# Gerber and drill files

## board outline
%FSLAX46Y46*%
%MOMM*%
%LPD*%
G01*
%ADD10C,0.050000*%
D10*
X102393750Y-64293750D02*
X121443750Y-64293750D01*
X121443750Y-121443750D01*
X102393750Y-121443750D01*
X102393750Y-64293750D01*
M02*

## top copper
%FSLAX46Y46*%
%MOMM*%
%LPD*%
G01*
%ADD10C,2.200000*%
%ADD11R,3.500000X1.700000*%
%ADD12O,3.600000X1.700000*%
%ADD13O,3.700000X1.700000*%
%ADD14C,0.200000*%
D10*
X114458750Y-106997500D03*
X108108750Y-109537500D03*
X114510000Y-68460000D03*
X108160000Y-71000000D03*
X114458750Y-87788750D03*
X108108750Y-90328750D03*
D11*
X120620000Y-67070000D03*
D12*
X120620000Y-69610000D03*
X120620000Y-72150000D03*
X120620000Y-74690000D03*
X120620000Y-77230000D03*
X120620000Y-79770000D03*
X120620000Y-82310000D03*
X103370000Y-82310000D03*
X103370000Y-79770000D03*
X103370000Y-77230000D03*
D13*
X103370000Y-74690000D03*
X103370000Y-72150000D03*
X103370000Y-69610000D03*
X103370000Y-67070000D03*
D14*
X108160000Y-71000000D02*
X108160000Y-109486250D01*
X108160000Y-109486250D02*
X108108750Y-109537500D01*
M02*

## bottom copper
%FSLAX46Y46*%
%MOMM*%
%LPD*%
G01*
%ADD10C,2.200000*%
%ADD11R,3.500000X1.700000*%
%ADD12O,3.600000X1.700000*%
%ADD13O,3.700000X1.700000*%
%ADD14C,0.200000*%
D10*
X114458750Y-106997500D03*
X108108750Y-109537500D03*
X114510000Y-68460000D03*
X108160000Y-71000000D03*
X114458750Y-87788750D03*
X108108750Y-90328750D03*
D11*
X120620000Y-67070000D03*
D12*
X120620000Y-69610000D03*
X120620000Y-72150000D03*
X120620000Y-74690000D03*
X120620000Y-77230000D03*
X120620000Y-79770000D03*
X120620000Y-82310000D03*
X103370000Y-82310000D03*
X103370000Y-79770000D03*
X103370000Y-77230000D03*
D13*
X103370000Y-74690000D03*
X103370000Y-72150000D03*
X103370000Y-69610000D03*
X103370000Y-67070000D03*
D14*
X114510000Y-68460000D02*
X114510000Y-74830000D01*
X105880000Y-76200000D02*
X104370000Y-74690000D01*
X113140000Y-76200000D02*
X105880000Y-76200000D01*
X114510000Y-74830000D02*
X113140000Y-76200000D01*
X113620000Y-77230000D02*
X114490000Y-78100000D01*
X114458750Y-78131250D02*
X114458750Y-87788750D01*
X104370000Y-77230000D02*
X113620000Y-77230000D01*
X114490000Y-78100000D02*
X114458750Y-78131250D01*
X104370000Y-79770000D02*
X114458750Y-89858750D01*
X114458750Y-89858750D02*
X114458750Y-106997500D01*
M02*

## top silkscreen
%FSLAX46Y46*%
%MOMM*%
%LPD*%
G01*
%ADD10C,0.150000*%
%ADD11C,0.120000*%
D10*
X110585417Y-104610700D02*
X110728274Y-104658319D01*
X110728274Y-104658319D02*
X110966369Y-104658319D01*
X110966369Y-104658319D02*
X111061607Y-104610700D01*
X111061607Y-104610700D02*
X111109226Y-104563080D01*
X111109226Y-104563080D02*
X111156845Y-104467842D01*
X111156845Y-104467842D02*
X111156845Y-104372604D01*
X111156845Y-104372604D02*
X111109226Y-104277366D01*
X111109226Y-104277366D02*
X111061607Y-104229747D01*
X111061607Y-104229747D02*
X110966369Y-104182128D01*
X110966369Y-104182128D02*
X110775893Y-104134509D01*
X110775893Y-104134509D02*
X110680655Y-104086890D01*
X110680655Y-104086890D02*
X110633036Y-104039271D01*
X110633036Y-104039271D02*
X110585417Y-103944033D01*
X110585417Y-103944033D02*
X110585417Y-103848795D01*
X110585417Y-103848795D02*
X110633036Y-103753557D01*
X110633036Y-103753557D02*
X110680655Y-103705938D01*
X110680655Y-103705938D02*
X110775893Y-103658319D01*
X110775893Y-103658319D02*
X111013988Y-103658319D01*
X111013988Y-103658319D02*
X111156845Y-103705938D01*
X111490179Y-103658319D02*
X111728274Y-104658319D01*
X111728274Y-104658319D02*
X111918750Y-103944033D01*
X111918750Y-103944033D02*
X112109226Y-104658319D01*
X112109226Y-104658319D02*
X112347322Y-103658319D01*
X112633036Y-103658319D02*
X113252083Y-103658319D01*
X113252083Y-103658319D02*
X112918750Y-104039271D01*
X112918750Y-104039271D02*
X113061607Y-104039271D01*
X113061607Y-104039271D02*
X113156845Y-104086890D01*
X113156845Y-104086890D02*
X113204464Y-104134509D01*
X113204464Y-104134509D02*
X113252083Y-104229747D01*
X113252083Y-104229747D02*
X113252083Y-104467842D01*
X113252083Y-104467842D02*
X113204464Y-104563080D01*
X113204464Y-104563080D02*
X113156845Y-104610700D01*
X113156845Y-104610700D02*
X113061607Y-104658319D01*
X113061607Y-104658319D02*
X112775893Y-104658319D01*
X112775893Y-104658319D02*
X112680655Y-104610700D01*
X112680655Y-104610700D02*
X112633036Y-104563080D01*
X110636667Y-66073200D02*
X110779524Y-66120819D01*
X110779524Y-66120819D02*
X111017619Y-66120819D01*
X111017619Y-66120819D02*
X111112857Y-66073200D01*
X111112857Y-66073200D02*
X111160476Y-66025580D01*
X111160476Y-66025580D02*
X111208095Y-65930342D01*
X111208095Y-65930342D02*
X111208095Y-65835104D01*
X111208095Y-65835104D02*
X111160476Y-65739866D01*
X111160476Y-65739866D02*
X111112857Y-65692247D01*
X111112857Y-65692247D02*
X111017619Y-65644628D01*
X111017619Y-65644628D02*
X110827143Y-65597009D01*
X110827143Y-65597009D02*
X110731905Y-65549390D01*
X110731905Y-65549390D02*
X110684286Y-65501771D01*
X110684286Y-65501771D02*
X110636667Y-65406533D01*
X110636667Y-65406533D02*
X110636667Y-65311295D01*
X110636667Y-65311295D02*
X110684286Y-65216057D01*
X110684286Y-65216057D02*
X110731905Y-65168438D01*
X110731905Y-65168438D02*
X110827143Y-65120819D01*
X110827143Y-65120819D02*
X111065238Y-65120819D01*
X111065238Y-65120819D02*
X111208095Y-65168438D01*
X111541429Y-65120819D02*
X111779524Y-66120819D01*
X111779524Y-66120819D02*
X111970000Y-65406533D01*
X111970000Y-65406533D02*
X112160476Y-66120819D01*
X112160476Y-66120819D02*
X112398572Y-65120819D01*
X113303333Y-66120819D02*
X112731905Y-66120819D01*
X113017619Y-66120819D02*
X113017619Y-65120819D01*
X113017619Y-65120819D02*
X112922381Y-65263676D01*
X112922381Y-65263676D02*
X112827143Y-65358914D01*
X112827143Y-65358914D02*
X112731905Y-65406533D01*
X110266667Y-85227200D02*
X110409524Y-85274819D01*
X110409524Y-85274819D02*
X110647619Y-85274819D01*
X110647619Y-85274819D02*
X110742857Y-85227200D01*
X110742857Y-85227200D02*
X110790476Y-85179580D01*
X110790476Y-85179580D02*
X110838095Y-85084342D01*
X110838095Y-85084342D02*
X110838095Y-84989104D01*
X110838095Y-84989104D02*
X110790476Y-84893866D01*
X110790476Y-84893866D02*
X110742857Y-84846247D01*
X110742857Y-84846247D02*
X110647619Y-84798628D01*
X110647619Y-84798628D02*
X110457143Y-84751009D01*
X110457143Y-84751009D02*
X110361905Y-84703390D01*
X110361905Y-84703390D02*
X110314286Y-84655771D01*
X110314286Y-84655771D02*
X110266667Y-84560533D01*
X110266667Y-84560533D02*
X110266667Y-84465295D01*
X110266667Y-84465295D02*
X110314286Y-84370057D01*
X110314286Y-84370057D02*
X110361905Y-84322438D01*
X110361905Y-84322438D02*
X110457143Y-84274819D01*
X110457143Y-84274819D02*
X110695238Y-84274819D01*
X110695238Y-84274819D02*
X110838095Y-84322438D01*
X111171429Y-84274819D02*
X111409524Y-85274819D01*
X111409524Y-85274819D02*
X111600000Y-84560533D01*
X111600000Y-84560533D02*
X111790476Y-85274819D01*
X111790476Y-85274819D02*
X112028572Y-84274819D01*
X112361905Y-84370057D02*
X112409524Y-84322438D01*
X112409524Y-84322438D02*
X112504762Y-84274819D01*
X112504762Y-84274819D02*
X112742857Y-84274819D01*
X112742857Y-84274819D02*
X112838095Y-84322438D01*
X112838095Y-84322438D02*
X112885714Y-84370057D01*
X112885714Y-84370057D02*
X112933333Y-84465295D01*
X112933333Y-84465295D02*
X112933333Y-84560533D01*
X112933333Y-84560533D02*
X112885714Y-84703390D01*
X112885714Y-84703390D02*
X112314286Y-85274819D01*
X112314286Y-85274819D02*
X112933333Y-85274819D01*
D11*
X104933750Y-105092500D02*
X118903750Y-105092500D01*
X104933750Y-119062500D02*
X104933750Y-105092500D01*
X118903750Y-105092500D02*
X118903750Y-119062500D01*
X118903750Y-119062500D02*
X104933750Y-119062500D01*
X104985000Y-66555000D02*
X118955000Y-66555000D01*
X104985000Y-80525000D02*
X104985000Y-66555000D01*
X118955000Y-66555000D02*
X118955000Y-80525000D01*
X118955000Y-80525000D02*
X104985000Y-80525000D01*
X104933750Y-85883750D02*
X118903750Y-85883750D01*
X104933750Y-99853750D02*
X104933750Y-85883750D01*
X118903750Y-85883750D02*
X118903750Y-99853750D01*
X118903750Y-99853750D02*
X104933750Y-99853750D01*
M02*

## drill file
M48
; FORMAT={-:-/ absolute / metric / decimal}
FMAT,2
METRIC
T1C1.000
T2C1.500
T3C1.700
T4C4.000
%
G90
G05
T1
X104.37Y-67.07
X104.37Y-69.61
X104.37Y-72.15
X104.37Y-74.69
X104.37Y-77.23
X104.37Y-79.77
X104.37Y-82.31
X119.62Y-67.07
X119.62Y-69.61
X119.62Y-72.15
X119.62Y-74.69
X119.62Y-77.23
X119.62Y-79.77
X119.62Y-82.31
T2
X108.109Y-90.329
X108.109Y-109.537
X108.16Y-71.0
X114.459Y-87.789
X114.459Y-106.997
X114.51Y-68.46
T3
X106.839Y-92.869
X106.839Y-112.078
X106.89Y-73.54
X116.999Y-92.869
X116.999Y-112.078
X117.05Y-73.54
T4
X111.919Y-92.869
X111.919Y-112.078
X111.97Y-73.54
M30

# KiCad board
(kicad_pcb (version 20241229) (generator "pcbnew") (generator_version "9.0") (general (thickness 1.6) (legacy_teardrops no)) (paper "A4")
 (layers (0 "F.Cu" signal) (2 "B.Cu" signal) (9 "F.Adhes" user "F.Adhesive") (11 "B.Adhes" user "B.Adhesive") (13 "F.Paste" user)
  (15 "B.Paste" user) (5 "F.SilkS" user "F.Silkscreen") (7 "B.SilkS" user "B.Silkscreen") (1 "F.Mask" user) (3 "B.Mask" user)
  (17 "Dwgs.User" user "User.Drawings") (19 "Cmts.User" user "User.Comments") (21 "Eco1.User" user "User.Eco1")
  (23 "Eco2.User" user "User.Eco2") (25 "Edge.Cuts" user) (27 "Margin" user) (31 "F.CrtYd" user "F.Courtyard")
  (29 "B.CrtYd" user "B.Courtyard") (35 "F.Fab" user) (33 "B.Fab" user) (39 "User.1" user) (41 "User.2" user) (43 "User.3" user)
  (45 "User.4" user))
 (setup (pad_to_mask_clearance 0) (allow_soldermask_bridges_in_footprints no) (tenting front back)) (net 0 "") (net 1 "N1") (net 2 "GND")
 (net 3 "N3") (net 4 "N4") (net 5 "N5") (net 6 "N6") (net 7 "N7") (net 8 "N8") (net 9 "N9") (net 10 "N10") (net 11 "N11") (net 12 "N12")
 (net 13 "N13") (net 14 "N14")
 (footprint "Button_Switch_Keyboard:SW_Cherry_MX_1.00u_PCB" (layer "F.Cu") (at 114.45875 106.9975)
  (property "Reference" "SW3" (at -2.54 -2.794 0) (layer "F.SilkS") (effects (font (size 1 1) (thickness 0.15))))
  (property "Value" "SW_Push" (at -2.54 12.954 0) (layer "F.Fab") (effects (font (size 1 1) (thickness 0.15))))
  (fp_line (start -9.525 -1.905) (end 4.445 -1.905) (stroke (width 0.12) (type solid)) (layer "F.SilkS"))
  (fp_line (start -9.525 12.065) (end -9.525 -1.905) (stroke (width 0.12) (type solid)) (layer "F.SilkS"))
  (fp_line (start 4.445 -1.905) (end 4.445 12.065) (stroke (width 0.12) (type solid)) (layer "F.SilkS"))
  (fp_line (start 4.445 12.065) (end -9.525 12.065) (stroke (width 0.12) (type solid)) (layer "F.SilkS"))
  (pad "" np_thru_hole circle (at -7.62 5.08) (size 1.7 1.7) (drill 1.7) (layers "*.Cu" "*.Mask"))
  (pad "" np_thru_hole circle (at -2.54 5.08) (size 4 4) (drill 4) (layers "*.Cu" "*.Mask"))
  (pad "" np_thru_hole circle (at 2.54 5.08) (size 1.7 1.7) (drill 1.7) (layers "*.Cu" "*.Mask"))
  (pad "1" thru_hole circle (at 0 0) (size 2.2 2.2) (drill 1.5) (layers "*.Cu" "*.Mask") (remove_unused_layers no) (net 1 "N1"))
  (pad "2" thru_hole circle (at -6.35 2.54) (size 2.2 2.2) (drill 1.5) (layers "*.Cu" "*.Mask") (remove_unused_layers no) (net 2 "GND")))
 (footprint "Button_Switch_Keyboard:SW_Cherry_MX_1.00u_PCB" (layer "F.Cu") (at 114.51 68.46)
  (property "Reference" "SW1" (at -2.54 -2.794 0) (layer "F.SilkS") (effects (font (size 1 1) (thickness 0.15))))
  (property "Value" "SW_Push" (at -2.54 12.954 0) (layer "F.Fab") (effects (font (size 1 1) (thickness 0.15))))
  (fp_line (start -9.525 -1.905) (end 4.445 -1.905) (stroke (width 0.12) (type solid)) (layer "F.SilkS"))
  (fp_line (start -9.525 12.065) (end -9.525 -1.905) (stroke (width 0.12) (type solid)) (layer "F.SilkS"))
  (fp_line (start 4.445 -1.905) (end 4.445 12.065) (stroke (width 0.12) (type solid)) (layer "F.SilkS"))
  (fp_line (start 4.445 12.065) (end -9.525 12.065) (stroke (width 0.12) (type solid)) (layer "F.SilkS"))
  (pad "" np_thru_hole circle (at -7.62 5.08) (size 1.7 1.7) (drill 1.7) (layers "*.Cu" "*.Mask"))
  (pad "" np_thru_hole circle (at -2.54 5.08) (size 4 4) (drill 4) (layers "*.Cu" "*.Mask"))
  (pad "" np_thru_hole circle (at 2.54 5.08) (size 1.7 1.7) (drill 1.7) (layers "*.Cu" "*.Mask"))
  (pad "1" thru_hole circle (at 0 0) (size 2.2 2.2) (drill 1.5) (layers "*.Cu" "*.Mask") (remove_unused_layers no) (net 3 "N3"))
  (pad "2" thru_hole circle (at -6.35 2.54) (size 2.2 2.2) (drill 1.5) (layers "*.Cu" "*.Mask") (remove_unused_layers no) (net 2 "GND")))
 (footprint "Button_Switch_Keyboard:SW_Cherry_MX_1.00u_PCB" (layer "F.Cu") (at 114.45875 87.78875)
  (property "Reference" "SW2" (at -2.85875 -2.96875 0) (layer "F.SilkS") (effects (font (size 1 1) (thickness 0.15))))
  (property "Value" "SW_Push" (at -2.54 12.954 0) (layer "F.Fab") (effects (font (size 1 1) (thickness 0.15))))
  (fp_line (start -9.525 -1.905) (end 4.445 -1.905) (stroke (width 0.12) (type solid)) (layer "F.SilkS"))
  (fp_line (start -9.525 12.065) (end -9.525 -1.905) (stroke (width 0.12) (type solid)) (layer "F.SilkS"))
  (fp_line (start 4.445 -1.905) (end 4.445 12.065) (stroke (width 0.12) (type solid)) (layer "F.SilkS"))
  (fp_line (start 4.445 12.065) (end -9.525 12.065) (stroke (width 0.12) (type solid)) (layer "F.SilkS"))
  (pad "" np_thru_hole circle (at -7.62 5.08) (size 1.7 1.7) (drill 1.7) (layers "*.Cu" "*.Mask"))
  (pad "" np_thru_hole circle (at -2.54 5.08) (size 4 4) (drill 4) (layers "*.Cu" "*.Mask"))
  (pad "" np_thru_hole circle (at 2.54 5.08) (size 1.7 1.7) (drill 1.7) (layers "*.Cu" "*.Mask"))
  (pad "1" thru_hole circle (at 0 0) (size 2.2 2.2) (drill 1.5) (layers "*.Cu" "*.Mask") (remove_unused_layers no) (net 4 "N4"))
  (pad "2" thru_hole circle (at -6.35 2.54) (size 2.2 2.2) (drill 1.5) (layers "*.Cu" "*.Mask") (remove_unused_layers no) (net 2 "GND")))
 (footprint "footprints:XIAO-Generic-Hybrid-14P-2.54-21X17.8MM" (layer "B.Cu") (at 111.995 74.69 180)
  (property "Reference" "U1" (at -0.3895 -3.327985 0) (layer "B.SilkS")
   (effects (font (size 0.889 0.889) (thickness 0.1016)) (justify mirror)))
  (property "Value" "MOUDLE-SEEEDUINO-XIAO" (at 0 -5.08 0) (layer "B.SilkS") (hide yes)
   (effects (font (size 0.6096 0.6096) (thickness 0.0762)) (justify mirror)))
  (pad "1" thru_hole rect (at -7.625 7.62 180) (size 3.5 1.7) (drill 1 (offset -1 0)) (layers "*.Cu" "*.Mask") (remove_unused_layers no)
   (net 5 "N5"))
  (pad "2" thru_hole oval (at -7.625 5.08 180) (size 3.6 1.7) (drill 1 (offset -1 0)) (layers "*.Cu" "*.Mask") (remove_unused_layers no)
   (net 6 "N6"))
  (pad "3" thru_hole oval (at -7.625 2.54 180) (size 3.6 1.7) (drill 1 (offset -1 0)) (layers "*.Cu" "*.Mask") (remove_unused_layers no)
   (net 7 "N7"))
  (pad "4" thru_hole oval (at -7.625 0 180) (size 3.6 1.7) (drill 1 (offset -1 0)) (layers "*.Cu" "*.Mask") (remove_unused_layers no)
   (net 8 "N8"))
  (pad "5" thru_hole oval (at -7.625 -2.54 180) (size 3.6 1.7) (drill 1 (offset -1 0)) (layers "*.Cu" "*.Mask") (remove_unused_layers no)
   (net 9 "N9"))
  (pad "6" thru_hole oval (at -7.625 -5.08) (size 3.6 1.7) (drill 1 (offset 1 0)) (layers "*.Cu" "*.Mask") (remove_unused_layers no)
   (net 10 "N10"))
  (pad "7" thru_hole oval (at -7.625 -7.62 180) (size 3.6 1.7) (drill 1 (offset -1 0)) (layers "*.Cu" "*.Mask") (remove_unused_layers no)
   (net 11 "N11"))
  (pad "8" thru_hole oval (at 7.625 -7.62 180) (size 3.6 1.7) (drill 1 (offset 1 0)) (layers "*.Cu" "*.Mask") (remove_unused_layers no)
   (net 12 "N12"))
  (pad "9" thru_hole oval (at 7.625 -5.08 180) (size 3.6 1.7) (drill 1 (offset 1 0)) (layers "*.Cu" "*.Mask") (remove_unused_layers no)
   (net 1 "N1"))
  (pad "10" thru_hole oval (at 7.625 -2.54 180) (size 3.6 1.7) (drill 1 (offset 1 0)) (layers "*.Cu" "*.Mask") (remove_unused_layers no)
   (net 4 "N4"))
  (pad "11" thru_hole oval (at 7.625 0 180) (size 3.7 1.7) (drill 1 (offset 1 0)) (layers "*.Cu" "*.Mask") (remove_unused_layers no)
   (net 3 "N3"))
  (pad "12" thru_hole oval (at 7.625 2.54 180) (size 3.7 1.7) (drill 1 (offset 1 0)) (layers "*.Cu" "*.Mask") (remove_unused_layers no)
   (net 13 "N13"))
  (pad "13" thru_hole oval (at 7.625 5.08 180) (size 3.7 1.7) (drill 1 (offset 1 0)) (layers "*.Cu" "*.Mask") (remove_unused_layers no)
   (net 2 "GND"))
  (pad "14" thru_hole oval (at 7.625 7.62 180) (size 3.7 1.7) (drill 1 (offset 1 0)) (layers "*.Cu" "*.Mask") (remove_unused_layers no)
   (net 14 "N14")))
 (gr_rect (start 102.39375 64.29375) (end 121.44375 121.44375) (stroke (width 0.05) (type default)) (fill no) (layer "Edge.Cuts"))
 (segment (start 108.16 71) (end 108.16 109.48625) (width 0.2) (layer "F.Cu") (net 2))
 (segment (start 108.16 109.48625) (end 108.10875 109.5375) (width 0.2) (layer "F.Cu") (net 2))
 (segment (start 114.51 68.46) (end 114.51 74.83) (width 0.2) (layer "B.Cu") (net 3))
 (segment (start 105.88 76.2) (end 104.37 74.69) (width 0.2) (layer "B.Cu") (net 3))
 (segment (start 113.14 76.2) (end 105.88 76.2) (width 0.2) (layer "B.Cu") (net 3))
 (segment (start 114.51 74.83) (end 113.14 76.2) (width 0.2) (layer "B.Cu") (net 3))
 (segment (start 113.62 77.23) (end 114.49 78.1) (width 0.2) (layer "B.Cu") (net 4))
 (segment (start 114.45875 78.13125) (end 114.45875 87.78875) (width 0.2) (layer "B.Cu") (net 4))
 (segment (start 104.37 77.23) (end 113.62 77.23) (width 0.2) (layer "B.Cu") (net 4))
 (segment (start 114.49 78.1) (end 114.45875 78.13125) (width 0.2) (layer "B.Cu") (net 4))
 (segment (start 104.37 79.77) (end 114.45875 89.85875) (width 0.2) (layer "B.Cu") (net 1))
 (segment (start 114.45875 89.85875) (end 114.45875 106.9975) (width 0.2) (layer "B.Cu") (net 1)))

